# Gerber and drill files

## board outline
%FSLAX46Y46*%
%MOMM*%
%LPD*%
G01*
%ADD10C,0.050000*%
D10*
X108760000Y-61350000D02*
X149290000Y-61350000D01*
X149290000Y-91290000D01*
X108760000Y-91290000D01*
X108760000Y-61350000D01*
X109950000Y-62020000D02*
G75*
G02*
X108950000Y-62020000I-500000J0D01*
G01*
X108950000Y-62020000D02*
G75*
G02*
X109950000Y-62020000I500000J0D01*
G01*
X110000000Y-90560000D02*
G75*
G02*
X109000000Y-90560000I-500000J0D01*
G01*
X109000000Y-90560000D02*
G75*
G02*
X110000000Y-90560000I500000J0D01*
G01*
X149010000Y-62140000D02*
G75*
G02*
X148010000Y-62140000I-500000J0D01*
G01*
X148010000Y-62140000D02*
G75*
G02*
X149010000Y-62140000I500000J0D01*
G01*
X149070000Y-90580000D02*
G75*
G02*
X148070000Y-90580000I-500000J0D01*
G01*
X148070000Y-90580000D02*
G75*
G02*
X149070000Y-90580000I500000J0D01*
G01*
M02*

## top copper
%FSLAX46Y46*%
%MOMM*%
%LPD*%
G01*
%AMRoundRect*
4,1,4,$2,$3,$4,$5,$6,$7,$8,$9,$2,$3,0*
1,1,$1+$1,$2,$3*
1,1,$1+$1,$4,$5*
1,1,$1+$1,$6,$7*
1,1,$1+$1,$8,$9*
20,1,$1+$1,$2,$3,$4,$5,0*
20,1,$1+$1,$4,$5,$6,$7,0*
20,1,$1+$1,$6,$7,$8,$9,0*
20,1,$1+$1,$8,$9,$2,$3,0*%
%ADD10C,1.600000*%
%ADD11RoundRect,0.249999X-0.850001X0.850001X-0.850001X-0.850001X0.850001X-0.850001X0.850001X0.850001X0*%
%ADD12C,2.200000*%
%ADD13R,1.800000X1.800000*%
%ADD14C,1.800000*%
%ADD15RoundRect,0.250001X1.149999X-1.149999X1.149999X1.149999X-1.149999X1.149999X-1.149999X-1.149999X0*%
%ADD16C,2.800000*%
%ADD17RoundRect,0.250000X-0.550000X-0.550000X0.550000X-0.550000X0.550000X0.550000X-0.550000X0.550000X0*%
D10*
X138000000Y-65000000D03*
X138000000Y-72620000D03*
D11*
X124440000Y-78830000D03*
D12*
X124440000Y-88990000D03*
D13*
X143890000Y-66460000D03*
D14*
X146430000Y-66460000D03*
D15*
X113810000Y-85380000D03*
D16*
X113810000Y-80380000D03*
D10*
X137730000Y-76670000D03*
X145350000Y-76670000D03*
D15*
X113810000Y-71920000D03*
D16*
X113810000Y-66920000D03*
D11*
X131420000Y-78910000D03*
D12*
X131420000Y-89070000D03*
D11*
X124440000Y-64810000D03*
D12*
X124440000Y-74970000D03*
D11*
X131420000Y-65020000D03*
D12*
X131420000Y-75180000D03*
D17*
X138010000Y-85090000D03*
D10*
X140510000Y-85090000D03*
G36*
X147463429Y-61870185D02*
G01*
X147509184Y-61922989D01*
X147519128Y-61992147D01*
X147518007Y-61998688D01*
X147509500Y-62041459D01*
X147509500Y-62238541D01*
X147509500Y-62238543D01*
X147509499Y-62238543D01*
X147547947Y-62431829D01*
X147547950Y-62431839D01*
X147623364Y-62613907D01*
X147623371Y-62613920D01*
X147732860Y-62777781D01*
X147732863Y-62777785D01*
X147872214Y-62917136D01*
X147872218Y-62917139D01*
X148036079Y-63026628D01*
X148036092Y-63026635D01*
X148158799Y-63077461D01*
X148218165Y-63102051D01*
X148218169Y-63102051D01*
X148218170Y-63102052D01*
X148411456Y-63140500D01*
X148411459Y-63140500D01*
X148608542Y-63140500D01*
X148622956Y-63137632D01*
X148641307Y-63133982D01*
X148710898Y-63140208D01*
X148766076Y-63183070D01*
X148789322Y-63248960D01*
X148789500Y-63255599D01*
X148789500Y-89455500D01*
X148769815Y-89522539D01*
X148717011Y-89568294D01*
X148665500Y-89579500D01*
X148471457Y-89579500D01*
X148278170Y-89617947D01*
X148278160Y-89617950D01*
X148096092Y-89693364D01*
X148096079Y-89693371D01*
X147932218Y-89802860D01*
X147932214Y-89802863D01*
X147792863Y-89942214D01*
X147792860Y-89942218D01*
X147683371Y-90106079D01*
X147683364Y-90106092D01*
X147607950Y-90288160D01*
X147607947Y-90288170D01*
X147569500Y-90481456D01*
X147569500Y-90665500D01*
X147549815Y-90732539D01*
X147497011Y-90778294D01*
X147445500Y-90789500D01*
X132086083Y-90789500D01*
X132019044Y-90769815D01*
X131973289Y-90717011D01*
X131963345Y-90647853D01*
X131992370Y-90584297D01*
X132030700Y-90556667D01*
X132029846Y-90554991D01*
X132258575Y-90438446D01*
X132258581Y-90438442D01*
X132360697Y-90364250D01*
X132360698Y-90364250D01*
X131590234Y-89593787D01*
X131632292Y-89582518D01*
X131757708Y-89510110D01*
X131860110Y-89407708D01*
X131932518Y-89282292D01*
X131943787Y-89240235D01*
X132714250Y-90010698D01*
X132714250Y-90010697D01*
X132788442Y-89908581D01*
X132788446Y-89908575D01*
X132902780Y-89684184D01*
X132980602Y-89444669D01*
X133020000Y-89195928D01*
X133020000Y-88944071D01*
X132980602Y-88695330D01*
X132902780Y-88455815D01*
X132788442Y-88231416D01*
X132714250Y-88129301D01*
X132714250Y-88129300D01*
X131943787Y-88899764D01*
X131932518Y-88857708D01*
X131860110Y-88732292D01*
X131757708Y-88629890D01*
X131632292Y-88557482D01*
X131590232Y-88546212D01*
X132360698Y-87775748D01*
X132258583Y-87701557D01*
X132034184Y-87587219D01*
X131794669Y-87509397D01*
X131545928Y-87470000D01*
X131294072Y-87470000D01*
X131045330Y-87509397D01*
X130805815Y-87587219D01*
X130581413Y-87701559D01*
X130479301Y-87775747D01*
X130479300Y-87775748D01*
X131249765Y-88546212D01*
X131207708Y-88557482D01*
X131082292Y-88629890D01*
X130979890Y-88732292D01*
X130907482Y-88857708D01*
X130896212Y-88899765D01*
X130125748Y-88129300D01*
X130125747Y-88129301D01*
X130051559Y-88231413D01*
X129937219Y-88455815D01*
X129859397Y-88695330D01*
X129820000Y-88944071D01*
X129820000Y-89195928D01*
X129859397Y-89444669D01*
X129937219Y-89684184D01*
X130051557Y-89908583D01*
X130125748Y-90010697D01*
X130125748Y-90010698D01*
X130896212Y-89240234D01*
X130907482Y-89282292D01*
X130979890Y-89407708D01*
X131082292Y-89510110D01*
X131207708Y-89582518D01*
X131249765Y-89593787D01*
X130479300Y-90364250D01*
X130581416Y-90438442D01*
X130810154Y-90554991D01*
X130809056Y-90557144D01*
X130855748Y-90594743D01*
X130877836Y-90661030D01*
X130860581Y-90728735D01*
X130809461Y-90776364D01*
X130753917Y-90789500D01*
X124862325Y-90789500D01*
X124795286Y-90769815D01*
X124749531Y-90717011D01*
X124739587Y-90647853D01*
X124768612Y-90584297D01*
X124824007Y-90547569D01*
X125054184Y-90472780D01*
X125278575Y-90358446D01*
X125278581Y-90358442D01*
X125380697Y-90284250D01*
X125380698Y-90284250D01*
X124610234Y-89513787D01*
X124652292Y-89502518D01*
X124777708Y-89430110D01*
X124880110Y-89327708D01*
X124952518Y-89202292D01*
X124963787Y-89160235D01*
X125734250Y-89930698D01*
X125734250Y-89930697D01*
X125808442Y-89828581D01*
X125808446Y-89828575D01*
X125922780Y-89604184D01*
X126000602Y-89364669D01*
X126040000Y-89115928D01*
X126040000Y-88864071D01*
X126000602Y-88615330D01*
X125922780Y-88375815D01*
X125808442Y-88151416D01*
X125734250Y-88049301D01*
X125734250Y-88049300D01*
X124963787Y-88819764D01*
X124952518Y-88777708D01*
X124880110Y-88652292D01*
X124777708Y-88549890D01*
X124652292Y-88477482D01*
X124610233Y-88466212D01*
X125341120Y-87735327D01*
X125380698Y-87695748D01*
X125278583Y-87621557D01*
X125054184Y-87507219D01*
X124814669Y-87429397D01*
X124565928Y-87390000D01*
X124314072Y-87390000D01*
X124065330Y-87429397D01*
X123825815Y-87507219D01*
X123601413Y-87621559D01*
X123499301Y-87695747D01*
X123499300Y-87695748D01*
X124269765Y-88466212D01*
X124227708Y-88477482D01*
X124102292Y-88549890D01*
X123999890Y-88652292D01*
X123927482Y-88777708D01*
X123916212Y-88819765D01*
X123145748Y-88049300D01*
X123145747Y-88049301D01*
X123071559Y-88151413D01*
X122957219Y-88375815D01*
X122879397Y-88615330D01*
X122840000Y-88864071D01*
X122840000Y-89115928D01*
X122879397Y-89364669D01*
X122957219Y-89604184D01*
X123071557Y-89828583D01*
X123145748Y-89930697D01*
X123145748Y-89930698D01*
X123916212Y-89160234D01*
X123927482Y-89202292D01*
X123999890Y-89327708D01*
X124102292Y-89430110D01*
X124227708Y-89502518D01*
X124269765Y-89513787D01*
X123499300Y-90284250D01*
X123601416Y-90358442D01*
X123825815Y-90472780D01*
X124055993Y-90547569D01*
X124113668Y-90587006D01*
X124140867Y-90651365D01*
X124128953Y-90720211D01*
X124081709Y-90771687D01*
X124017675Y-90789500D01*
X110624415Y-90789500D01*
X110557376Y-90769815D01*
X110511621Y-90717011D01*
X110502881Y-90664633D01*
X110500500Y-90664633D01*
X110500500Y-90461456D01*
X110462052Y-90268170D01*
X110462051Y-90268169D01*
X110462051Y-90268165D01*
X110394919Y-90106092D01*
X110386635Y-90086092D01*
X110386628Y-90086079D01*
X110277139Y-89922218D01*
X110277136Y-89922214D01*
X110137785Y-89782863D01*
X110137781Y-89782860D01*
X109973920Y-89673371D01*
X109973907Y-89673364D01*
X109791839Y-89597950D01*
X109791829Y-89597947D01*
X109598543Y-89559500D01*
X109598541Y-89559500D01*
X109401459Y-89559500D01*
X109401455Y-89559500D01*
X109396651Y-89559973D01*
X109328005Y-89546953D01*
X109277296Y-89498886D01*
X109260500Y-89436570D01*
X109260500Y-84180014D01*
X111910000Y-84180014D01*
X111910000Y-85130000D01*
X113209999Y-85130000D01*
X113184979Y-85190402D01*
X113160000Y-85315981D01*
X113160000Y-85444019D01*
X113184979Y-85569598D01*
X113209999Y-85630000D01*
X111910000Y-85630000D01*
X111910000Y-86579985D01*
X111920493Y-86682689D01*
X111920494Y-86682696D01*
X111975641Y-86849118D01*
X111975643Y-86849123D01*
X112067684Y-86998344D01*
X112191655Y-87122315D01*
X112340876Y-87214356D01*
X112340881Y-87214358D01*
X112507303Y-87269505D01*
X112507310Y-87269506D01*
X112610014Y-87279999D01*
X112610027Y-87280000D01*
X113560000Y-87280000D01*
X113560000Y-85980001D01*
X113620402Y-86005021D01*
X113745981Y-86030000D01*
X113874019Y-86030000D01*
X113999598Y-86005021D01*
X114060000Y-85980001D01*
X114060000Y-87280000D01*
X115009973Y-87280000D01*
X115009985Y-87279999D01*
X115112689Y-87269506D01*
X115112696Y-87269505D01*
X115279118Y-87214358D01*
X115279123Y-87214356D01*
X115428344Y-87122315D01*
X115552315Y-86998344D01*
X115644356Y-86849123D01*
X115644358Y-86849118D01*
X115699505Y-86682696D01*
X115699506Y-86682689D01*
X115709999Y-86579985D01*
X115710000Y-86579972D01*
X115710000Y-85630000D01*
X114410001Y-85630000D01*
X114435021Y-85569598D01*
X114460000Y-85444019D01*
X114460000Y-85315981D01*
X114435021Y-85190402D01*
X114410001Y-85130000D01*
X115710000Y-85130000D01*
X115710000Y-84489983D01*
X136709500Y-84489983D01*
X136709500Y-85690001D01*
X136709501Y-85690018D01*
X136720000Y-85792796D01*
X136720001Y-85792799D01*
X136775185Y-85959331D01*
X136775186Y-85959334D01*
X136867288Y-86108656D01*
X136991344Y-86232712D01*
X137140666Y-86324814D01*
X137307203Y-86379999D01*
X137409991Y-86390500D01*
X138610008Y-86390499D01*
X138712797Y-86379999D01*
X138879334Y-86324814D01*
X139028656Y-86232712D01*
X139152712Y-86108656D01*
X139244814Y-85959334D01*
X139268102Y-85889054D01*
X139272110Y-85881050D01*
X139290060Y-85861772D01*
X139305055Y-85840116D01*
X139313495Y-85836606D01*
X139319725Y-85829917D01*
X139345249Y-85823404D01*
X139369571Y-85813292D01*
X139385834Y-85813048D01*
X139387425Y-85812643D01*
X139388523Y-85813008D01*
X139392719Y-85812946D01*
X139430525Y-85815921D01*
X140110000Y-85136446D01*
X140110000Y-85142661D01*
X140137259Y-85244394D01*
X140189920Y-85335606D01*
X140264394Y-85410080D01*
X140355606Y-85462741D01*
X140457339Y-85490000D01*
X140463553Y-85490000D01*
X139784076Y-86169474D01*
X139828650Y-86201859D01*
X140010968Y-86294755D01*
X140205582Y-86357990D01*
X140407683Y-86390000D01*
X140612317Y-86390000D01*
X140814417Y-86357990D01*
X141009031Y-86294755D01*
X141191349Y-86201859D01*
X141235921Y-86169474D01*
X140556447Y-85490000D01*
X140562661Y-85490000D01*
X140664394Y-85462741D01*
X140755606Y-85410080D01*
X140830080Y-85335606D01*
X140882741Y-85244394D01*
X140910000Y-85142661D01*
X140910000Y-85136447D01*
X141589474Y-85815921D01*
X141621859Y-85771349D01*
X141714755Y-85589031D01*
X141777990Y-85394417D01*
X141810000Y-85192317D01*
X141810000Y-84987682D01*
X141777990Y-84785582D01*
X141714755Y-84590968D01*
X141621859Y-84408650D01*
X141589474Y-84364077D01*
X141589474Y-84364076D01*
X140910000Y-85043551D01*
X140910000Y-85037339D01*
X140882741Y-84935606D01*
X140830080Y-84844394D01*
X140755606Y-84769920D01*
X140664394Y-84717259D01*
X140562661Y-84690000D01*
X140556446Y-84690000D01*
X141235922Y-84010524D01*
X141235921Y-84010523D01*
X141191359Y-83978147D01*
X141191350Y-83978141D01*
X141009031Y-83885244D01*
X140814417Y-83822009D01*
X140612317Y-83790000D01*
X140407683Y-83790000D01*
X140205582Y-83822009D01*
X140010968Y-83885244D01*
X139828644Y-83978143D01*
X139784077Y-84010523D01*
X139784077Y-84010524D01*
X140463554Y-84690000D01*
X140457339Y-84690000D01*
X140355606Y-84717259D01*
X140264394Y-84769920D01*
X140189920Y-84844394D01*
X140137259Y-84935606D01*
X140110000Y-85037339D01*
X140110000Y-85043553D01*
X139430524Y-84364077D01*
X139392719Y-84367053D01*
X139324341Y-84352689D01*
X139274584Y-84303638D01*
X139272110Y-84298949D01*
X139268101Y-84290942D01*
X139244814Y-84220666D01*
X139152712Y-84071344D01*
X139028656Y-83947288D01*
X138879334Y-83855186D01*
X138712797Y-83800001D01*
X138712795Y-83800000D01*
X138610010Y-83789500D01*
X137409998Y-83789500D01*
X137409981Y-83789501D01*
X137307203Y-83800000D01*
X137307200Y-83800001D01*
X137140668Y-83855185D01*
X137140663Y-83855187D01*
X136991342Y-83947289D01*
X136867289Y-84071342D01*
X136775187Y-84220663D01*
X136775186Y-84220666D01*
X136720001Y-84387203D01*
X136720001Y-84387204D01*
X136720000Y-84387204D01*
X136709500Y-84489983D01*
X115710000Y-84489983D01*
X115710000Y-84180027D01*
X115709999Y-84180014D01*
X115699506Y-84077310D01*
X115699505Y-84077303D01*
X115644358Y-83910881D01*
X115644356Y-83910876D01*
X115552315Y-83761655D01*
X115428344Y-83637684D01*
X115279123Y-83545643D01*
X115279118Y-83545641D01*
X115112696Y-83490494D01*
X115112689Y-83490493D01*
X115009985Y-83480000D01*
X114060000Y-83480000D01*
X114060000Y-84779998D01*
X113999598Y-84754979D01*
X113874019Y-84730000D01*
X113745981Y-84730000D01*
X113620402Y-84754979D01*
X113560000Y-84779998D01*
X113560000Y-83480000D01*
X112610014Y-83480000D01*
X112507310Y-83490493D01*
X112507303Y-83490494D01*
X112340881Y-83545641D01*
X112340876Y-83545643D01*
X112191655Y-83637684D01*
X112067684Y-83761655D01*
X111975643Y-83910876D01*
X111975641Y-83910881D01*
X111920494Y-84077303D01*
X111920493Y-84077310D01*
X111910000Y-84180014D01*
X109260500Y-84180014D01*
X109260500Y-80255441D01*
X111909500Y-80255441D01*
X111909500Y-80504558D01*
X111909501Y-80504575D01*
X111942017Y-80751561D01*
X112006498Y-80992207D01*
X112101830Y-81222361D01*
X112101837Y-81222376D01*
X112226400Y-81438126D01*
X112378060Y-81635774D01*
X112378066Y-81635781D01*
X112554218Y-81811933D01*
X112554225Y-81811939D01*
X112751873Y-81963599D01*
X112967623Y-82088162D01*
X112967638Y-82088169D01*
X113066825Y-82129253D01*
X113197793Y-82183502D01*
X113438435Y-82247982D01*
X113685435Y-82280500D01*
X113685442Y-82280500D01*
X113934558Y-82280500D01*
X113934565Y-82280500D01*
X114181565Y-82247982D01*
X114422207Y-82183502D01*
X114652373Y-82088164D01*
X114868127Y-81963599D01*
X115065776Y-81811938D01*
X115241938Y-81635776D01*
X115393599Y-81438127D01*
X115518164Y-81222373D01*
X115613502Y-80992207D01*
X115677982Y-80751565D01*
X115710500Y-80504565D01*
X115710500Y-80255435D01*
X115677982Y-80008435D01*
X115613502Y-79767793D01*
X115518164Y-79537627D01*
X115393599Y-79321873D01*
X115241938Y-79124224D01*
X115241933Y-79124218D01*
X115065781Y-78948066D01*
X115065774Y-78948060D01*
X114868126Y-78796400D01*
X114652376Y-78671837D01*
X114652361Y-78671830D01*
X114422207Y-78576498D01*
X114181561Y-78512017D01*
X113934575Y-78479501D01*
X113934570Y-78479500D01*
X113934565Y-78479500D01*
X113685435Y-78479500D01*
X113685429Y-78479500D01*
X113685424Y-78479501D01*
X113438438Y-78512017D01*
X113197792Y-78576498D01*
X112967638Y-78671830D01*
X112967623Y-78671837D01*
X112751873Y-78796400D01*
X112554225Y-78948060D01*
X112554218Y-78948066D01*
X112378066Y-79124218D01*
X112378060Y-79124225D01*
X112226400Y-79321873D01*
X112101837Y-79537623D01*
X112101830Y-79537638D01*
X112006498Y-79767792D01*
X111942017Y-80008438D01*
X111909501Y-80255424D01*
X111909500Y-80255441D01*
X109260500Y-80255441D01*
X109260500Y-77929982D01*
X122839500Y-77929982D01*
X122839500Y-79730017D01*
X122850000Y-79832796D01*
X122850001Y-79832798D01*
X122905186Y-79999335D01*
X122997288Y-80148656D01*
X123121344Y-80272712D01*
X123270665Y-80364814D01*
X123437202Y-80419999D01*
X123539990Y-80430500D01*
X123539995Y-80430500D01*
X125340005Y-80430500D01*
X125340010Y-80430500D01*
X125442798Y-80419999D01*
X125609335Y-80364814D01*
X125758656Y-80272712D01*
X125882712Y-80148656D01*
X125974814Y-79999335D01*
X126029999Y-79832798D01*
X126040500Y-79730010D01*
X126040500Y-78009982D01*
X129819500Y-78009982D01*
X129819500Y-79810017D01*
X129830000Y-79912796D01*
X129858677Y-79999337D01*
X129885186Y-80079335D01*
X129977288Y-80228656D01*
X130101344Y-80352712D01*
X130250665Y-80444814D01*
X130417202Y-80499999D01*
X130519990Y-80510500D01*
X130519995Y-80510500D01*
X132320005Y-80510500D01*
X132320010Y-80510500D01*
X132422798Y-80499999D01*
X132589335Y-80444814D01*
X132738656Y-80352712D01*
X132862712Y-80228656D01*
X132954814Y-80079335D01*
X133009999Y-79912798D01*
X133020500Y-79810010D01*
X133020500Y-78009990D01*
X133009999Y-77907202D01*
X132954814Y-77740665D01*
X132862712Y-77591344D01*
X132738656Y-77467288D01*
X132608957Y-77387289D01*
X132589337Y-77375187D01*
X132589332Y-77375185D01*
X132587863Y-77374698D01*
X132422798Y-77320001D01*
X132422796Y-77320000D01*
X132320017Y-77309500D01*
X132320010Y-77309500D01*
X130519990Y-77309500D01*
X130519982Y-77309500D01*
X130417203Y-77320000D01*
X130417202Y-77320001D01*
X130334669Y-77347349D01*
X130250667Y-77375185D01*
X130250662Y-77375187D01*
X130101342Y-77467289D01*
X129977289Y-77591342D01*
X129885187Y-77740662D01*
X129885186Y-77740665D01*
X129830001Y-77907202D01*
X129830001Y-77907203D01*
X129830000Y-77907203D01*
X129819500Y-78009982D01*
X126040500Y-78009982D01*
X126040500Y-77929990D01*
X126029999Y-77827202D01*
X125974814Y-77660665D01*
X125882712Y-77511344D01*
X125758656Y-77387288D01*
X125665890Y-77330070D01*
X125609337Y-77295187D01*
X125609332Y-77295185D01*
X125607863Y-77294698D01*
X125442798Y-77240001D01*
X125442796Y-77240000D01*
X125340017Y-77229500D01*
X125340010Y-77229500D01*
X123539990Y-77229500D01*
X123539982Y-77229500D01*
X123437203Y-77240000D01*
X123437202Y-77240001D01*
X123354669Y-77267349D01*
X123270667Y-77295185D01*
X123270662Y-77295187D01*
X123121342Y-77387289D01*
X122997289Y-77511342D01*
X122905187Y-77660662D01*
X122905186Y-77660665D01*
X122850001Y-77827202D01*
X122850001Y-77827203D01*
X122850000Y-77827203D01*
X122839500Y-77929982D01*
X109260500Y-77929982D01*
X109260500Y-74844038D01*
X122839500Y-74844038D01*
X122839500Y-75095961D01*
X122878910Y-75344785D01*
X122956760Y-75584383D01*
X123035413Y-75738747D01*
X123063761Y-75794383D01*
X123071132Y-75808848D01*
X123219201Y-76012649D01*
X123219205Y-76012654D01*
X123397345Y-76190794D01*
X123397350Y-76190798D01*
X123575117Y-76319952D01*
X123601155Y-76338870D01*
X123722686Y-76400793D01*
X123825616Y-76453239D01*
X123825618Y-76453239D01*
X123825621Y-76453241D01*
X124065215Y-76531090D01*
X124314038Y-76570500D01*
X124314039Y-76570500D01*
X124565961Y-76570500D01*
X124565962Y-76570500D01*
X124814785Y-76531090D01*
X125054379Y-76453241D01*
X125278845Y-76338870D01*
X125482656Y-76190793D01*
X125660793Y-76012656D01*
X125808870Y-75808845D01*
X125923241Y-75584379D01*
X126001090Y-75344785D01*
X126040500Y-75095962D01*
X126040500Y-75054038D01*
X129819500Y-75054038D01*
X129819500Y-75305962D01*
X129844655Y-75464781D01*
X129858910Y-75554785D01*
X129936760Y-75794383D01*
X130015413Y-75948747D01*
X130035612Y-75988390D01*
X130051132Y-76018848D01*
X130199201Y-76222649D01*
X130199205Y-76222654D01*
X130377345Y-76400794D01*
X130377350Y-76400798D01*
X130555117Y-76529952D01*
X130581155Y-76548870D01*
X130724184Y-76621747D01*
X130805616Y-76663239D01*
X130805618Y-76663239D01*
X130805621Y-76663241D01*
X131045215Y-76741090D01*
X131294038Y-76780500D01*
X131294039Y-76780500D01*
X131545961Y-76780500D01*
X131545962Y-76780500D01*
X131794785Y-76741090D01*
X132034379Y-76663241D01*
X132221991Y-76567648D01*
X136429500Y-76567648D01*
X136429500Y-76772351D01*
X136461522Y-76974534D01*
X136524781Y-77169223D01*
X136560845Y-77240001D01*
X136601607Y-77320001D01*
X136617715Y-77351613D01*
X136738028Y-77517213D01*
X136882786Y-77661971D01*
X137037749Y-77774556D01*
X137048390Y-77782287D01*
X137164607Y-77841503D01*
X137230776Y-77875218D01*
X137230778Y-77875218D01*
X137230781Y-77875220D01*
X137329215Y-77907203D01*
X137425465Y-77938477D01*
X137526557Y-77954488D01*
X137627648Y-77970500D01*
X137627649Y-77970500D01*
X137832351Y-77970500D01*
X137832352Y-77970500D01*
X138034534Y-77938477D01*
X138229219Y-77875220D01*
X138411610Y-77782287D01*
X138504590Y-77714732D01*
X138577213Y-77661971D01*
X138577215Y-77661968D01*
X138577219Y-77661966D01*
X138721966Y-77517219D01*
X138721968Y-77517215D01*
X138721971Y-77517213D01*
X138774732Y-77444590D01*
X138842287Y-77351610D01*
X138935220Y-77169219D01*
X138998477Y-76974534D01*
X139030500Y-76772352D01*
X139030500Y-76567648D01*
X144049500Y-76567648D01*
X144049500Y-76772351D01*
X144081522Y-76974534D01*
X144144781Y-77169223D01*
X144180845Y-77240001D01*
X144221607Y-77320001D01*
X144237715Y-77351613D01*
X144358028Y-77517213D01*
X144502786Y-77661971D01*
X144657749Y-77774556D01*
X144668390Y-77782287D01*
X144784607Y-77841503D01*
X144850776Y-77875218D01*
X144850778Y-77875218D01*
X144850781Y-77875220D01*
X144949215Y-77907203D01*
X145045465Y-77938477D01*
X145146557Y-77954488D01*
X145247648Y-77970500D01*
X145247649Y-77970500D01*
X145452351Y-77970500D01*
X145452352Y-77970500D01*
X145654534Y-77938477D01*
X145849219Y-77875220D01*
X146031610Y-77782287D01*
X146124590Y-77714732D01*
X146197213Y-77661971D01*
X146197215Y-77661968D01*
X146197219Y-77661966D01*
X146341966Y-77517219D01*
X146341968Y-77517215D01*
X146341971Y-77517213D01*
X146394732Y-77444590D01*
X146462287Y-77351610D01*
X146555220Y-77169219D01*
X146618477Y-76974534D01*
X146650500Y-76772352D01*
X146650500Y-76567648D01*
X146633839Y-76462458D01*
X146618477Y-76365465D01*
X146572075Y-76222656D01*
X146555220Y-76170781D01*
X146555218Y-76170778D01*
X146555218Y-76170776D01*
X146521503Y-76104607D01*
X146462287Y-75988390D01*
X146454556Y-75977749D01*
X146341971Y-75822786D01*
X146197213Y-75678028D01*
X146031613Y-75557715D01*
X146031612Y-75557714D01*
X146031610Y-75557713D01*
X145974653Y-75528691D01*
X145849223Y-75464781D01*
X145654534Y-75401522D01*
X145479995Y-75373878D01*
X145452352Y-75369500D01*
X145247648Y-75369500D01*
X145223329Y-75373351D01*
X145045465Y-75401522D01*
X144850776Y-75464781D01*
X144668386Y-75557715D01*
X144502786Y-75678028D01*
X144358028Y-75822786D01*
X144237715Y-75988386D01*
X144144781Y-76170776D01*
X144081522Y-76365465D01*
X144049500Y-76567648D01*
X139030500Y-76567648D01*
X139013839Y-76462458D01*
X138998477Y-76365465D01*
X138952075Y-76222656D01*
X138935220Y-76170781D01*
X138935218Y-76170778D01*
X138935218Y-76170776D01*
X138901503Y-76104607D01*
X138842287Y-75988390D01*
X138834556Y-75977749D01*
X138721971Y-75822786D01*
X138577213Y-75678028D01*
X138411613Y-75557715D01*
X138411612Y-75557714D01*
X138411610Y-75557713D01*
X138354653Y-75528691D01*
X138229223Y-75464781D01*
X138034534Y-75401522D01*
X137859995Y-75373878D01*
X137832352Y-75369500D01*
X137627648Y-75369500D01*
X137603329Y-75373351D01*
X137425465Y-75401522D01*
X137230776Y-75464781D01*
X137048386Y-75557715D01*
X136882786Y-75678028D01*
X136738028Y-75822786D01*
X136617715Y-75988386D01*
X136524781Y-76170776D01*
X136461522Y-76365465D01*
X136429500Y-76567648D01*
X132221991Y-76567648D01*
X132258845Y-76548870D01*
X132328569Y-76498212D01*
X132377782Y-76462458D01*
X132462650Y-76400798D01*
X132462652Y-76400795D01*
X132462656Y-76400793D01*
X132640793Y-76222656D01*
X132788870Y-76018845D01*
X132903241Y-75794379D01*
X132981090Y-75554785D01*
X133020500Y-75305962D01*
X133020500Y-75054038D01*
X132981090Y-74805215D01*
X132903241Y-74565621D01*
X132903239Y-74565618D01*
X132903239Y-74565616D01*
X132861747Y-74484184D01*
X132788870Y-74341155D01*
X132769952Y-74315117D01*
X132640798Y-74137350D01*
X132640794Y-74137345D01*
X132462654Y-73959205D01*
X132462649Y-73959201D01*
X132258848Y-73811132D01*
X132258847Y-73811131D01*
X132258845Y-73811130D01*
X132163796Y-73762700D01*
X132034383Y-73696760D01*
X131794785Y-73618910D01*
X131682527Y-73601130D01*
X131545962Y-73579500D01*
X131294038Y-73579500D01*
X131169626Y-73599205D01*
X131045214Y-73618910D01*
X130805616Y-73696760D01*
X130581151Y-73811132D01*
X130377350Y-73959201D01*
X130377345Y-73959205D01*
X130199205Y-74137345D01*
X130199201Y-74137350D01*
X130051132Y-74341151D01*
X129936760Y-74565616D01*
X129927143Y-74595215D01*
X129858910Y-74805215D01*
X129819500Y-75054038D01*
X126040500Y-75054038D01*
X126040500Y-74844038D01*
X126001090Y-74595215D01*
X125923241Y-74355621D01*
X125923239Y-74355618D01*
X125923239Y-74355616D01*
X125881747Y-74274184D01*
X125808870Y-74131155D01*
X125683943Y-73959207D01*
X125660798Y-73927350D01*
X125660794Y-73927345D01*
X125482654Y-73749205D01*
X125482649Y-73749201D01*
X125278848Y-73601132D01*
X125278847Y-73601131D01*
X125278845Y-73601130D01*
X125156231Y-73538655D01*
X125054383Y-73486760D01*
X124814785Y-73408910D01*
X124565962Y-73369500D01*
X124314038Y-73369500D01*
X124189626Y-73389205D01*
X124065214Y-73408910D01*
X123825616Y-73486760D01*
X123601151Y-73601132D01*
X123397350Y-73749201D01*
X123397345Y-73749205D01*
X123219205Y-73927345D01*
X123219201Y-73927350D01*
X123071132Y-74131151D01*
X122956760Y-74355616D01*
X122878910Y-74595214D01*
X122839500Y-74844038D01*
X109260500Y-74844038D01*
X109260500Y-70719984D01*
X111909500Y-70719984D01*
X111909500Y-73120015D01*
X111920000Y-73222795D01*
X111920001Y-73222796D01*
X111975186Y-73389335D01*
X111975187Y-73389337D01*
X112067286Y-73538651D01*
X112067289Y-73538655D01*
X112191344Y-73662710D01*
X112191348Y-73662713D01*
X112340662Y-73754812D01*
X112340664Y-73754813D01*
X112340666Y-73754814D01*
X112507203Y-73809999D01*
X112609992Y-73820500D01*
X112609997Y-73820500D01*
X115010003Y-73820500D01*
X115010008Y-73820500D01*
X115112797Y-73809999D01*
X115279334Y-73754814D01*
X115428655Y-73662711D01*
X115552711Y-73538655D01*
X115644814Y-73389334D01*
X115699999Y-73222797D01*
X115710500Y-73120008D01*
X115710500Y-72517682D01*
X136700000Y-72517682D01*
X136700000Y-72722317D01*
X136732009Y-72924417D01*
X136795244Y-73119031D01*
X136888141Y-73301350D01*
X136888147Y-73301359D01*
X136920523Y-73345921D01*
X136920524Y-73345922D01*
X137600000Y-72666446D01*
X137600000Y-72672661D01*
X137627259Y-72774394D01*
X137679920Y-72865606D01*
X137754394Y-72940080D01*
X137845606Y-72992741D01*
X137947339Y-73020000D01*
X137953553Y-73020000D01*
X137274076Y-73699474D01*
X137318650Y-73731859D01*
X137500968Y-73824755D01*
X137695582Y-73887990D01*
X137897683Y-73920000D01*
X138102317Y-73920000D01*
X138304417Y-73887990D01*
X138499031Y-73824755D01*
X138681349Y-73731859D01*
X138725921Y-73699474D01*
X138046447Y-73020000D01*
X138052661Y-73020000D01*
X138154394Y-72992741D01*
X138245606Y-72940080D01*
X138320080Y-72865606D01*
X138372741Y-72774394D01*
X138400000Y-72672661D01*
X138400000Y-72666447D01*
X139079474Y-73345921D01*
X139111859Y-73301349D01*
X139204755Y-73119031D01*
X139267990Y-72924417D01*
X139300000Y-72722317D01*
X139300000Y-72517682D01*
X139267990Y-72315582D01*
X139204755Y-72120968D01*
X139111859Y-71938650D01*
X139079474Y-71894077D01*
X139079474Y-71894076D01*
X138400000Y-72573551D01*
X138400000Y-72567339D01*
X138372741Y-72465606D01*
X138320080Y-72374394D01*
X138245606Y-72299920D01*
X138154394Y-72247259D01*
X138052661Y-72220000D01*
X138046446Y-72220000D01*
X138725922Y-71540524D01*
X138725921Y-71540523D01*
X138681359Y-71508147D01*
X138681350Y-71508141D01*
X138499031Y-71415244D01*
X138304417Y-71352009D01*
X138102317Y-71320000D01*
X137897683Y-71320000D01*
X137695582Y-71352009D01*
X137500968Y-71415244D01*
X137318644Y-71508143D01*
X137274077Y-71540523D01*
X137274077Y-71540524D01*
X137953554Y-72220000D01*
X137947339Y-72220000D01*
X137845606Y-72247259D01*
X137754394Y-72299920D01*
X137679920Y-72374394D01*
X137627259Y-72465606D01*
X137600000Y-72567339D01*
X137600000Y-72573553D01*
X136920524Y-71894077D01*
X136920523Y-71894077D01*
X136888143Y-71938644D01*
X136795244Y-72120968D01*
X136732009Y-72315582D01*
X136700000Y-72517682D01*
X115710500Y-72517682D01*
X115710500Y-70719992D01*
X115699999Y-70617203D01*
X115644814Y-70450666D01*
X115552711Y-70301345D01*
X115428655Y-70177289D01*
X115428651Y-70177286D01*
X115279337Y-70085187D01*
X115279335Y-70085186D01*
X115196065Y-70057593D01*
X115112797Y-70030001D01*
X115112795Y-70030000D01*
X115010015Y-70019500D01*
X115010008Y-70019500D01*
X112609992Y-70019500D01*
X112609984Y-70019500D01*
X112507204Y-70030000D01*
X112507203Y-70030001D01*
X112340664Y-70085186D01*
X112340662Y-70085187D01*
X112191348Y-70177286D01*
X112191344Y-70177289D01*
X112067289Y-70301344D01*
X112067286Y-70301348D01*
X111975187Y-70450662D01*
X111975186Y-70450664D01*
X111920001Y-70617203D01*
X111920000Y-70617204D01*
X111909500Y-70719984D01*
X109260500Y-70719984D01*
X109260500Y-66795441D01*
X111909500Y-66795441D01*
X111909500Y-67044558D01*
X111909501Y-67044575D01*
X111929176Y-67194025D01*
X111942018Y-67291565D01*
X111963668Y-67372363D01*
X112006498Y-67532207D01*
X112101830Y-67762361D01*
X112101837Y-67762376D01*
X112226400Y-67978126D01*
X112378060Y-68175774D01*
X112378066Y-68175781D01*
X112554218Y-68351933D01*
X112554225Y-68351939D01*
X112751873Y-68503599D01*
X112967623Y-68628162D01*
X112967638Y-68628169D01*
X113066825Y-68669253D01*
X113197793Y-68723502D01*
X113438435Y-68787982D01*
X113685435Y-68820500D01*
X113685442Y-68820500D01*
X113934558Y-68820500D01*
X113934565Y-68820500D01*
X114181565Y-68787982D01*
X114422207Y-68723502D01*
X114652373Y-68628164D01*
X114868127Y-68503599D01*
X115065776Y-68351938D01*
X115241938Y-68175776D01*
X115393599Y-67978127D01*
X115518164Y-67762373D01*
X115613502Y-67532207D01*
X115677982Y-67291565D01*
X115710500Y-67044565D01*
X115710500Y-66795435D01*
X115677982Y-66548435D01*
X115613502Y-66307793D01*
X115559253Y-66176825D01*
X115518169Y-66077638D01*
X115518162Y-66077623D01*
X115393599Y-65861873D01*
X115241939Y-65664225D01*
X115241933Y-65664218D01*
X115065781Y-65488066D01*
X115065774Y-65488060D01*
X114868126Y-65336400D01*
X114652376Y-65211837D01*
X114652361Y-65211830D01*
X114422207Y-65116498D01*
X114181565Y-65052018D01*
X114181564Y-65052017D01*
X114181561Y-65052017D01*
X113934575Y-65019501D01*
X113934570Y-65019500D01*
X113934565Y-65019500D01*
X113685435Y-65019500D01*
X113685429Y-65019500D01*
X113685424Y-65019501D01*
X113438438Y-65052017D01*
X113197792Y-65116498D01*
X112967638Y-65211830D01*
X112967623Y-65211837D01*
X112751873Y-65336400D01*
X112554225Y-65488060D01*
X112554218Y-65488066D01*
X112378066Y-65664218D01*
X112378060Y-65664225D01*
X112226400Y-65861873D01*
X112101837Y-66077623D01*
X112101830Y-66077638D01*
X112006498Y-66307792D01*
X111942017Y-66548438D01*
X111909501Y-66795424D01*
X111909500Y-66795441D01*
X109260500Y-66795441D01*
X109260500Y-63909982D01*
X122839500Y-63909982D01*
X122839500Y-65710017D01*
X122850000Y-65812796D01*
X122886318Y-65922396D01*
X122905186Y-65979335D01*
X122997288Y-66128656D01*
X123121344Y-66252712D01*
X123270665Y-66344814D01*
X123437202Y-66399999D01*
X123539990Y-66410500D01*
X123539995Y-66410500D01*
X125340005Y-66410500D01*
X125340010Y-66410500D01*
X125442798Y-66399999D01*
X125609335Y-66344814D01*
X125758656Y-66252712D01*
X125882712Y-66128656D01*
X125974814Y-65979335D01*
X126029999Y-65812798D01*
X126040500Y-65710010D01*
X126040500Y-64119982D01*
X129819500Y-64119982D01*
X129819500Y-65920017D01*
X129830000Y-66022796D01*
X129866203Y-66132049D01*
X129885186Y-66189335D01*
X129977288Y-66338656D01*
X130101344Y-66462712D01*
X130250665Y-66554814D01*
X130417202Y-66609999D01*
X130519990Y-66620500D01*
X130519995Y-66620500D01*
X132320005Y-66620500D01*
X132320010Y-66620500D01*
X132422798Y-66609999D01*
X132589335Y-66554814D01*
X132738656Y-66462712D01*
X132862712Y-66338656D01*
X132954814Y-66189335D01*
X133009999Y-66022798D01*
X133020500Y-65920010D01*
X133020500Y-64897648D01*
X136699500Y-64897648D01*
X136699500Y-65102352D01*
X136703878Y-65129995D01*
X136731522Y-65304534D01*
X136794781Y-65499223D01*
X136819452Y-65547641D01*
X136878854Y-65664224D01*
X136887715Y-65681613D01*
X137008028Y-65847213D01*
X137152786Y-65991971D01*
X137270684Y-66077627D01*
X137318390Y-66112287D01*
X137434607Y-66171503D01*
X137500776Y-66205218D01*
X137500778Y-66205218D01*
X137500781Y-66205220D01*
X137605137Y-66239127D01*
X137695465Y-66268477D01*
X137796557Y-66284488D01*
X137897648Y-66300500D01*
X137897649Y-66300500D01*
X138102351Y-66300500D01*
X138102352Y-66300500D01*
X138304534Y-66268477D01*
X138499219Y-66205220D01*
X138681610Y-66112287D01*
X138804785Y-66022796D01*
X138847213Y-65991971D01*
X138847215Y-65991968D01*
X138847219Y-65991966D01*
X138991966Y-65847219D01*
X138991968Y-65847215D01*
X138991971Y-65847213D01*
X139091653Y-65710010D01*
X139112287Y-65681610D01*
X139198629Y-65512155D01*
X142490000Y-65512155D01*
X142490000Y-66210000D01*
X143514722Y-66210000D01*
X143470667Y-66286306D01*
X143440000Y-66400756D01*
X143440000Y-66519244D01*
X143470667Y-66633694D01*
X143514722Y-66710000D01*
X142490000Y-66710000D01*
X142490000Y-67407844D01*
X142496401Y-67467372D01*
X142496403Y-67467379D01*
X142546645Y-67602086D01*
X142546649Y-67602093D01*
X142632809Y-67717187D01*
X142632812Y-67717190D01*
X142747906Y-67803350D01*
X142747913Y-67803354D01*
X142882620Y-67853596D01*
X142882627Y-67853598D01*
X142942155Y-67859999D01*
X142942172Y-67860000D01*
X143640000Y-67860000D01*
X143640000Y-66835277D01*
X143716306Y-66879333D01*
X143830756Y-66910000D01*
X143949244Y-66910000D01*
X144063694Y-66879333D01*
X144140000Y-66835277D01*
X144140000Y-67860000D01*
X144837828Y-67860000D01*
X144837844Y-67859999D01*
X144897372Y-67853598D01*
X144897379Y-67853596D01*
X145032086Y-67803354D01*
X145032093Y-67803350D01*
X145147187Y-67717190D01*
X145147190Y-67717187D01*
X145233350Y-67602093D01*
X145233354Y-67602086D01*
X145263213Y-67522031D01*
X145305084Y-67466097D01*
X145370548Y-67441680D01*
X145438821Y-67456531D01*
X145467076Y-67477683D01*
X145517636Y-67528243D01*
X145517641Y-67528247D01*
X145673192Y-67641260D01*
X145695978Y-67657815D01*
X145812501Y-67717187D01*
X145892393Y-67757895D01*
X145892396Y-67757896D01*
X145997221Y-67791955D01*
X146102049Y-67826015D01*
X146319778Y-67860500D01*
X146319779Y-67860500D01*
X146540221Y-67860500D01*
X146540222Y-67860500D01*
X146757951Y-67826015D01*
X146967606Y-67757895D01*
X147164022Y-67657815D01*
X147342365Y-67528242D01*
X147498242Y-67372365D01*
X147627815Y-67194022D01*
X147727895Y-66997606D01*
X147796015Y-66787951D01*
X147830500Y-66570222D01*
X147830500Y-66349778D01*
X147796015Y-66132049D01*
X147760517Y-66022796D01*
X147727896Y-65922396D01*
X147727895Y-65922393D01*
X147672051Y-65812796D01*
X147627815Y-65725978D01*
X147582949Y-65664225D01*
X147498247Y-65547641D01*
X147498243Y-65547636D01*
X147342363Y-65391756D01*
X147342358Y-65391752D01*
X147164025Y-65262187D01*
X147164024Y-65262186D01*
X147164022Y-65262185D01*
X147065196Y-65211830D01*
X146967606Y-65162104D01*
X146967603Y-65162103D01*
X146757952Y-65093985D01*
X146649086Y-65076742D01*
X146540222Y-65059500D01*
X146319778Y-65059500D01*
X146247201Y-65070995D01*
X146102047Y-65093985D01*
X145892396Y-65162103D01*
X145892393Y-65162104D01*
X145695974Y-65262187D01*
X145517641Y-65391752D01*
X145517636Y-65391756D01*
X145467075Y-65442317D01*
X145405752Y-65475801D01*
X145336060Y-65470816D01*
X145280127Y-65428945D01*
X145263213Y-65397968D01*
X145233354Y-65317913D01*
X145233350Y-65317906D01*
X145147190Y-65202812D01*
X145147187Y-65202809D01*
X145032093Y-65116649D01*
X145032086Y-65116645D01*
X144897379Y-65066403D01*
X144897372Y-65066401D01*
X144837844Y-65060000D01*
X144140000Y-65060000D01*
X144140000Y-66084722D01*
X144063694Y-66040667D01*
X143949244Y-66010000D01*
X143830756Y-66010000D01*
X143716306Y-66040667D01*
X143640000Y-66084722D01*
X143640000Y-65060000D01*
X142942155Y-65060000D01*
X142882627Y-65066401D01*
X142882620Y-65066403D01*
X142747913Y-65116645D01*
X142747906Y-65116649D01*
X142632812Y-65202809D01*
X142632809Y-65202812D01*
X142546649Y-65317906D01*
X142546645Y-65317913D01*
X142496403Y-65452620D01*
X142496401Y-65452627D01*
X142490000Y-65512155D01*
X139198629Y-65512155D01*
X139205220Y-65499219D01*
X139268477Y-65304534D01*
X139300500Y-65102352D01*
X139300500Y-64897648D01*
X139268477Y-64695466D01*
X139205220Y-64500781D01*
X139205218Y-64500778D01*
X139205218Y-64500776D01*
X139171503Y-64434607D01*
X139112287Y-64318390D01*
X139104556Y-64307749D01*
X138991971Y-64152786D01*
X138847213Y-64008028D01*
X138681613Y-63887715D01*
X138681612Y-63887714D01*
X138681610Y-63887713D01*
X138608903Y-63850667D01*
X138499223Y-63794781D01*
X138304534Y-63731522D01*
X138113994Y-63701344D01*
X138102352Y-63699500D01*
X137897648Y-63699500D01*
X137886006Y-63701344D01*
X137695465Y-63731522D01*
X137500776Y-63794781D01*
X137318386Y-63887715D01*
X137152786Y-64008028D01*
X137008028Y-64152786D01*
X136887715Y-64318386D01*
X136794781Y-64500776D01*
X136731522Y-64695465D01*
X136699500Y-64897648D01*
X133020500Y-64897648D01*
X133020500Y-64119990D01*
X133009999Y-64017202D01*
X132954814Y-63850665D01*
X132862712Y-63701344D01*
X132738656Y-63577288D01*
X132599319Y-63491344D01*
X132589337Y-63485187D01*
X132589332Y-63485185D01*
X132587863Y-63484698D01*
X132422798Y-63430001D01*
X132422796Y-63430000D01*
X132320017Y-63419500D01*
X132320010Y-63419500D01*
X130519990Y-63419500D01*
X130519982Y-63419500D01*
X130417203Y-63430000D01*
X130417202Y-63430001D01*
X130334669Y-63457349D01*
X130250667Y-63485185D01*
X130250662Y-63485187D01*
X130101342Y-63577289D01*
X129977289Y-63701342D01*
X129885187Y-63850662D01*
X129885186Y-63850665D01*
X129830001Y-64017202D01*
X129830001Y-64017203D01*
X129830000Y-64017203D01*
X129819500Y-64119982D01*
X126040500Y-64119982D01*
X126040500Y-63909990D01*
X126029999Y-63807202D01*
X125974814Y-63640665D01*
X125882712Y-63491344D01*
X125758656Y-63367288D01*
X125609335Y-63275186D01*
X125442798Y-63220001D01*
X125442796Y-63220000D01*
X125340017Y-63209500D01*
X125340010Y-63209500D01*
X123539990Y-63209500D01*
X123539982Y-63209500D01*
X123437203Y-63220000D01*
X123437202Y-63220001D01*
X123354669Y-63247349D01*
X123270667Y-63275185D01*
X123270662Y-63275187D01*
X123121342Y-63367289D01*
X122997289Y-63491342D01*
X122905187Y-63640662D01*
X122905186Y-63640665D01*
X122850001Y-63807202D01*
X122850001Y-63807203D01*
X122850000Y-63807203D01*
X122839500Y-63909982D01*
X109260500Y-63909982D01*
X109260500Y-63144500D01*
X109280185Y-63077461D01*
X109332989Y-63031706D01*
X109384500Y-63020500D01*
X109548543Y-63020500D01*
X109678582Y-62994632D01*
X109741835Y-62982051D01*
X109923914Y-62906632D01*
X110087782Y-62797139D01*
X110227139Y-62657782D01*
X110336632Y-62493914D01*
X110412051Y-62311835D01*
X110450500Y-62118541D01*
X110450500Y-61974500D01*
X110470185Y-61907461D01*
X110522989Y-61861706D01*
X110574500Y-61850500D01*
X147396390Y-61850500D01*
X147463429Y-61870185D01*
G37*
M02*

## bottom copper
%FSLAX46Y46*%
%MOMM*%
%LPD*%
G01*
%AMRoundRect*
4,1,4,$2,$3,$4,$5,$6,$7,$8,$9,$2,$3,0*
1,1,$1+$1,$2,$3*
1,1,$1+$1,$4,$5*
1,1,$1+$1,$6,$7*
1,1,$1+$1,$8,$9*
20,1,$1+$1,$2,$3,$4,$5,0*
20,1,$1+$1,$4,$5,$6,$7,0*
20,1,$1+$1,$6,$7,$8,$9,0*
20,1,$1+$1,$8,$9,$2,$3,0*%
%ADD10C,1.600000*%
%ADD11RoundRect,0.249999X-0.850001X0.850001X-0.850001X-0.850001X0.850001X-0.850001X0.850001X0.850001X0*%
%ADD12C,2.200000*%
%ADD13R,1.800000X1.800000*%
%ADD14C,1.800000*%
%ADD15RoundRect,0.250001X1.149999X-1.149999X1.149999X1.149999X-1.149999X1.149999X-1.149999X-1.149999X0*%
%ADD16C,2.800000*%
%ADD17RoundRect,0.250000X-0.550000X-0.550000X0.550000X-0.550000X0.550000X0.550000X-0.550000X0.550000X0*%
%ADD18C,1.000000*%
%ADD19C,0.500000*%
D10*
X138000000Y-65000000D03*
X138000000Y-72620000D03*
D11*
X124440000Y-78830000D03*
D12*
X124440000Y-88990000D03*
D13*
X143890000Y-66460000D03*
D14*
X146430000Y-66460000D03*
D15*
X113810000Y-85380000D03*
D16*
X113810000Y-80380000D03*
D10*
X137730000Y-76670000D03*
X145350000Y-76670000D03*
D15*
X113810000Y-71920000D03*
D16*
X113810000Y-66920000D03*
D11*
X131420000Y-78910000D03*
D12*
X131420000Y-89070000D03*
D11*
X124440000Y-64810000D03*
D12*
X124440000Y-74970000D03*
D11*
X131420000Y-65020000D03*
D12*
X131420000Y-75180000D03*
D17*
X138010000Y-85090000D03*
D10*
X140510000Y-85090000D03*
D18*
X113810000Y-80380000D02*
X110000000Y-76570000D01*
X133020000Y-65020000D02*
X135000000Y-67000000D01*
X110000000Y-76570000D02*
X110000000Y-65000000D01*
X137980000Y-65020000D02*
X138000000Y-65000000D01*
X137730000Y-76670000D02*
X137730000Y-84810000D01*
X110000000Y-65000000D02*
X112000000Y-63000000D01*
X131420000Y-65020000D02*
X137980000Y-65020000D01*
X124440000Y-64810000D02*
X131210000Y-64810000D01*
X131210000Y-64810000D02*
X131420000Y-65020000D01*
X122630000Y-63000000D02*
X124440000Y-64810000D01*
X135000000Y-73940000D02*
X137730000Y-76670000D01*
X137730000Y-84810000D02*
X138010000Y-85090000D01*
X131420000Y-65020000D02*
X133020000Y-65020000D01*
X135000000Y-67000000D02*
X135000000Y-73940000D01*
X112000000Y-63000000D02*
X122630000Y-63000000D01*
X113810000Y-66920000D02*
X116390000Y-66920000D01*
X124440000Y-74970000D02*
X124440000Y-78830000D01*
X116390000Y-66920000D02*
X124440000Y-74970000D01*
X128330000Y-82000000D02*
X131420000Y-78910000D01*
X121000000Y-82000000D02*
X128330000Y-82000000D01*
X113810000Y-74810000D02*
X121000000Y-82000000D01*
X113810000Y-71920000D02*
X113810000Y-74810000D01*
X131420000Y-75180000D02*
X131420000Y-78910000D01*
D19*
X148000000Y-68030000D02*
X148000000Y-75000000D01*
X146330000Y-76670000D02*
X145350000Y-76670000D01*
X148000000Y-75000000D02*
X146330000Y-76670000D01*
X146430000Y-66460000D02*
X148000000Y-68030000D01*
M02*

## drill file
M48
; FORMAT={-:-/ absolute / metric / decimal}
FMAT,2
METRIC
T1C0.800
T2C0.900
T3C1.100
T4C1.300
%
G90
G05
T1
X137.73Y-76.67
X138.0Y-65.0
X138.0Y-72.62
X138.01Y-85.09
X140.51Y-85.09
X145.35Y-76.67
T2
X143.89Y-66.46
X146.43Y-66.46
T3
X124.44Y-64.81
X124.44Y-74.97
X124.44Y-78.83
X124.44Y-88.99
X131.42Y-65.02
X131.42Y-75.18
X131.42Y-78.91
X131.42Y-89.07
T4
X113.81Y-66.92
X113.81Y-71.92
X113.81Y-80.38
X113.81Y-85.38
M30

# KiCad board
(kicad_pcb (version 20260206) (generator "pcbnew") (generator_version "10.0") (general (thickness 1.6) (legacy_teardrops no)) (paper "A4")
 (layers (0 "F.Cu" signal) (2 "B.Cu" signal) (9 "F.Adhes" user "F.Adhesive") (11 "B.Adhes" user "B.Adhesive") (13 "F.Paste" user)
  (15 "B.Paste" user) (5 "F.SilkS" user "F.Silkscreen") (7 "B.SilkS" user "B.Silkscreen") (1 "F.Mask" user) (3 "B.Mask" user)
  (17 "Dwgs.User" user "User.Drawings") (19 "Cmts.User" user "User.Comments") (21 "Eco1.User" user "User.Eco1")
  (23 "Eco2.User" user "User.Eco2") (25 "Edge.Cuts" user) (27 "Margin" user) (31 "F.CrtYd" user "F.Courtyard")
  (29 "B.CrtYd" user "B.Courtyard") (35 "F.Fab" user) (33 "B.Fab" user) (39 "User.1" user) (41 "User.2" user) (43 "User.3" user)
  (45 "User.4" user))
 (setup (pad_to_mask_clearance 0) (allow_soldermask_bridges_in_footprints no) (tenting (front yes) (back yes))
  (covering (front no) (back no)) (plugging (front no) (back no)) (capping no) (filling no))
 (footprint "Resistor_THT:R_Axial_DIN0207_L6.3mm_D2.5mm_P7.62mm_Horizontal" (layer "F.Cu") (at 138 65 -90)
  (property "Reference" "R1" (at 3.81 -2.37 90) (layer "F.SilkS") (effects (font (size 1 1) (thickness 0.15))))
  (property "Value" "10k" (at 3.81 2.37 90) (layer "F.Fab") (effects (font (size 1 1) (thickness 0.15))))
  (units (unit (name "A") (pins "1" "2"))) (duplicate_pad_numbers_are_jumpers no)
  (pad "1" thru_hole circle (at 0 0 270) (size 1.6 1.6) (drill 0.8) (layers "*.Cu" "*.Mask") (remove_unused_layers no) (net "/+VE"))
  (pad "2" thru_hole circle (at 7.62 0 270) (size 1.6 1.6) (drill 0.8) (layers "*.Cu" "*.Mask") (remove_unused_layers no) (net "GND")))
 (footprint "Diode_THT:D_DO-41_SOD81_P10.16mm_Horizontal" (layer "F.Cu") (at 124.44 78.83 -90)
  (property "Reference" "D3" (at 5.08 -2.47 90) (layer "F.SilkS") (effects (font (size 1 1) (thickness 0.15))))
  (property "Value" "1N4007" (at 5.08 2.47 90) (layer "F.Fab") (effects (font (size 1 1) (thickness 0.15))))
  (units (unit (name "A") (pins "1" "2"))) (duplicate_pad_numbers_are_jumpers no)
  (pad "1" thru_hole roundrect (at 0 0 270) (size 2.2 2.2) (drill 1.1) (layers "*.Cu" "*.Mask") (remove_unused_layers no)
   (roundrect_rratio 0.113636) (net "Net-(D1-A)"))
  (pad "2" thru_hole circle (at 10.16 0 270) (size 2.2 2.2) (drill 1.1) (layers "*.Cu" "*.Mask") (remove_unused_layers no) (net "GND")))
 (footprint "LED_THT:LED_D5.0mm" (layer "F.Cu") (at 143.89 66.46)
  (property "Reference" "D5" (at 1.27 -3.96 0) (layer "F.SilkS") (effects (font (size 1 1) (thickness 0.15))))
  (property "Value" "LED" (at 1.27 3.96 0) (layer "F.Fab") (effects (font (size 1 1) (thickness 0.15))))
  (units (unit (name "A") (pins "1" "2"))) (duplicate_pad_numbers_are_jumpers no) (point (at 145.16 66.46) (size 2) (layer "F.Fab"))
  (pad "1" thru_hole rect (at 0 0) (size 1.8 1.8) (drill 0.9) (layers "*.Cu" "*.Mask") (remove_unused_layers no) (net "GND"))
  (pad "2" thru_hole circle (at 2.54 0) (size 1.8 1.8) (drill 0.9) (layers "*.Cu" "*.Mask") (remove_unused_layers no) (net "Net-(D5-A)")))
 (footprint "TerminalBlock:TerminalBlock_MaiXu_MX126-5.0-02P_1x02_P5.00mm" (layer "F.Cu") (at 113.81 85.38 90)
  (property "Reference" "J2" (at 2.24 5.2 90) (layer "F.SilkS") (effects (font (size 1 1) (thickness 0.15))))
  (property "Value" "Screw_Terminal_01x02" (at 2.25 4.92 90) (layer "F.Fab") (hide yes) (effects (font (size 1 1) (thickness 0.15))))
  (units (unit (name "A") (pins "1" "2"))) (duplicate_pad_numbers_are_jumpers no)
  (pad "1" thru_hole roundrect (at 0 0 90) (size 2.8 2.8) (drill 1.3) (layers "*.Cu" "*.Mask") (remove_unused_layers no)
   (roundrect_rratio 0.089286) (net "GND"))
  (pad "2" thru_hole circle (at 5 0 90) (size 2.8 2.8) (drill 1.3) (layers "*.Cu" "*.Mask") (remove_unused_layers no) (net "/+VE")))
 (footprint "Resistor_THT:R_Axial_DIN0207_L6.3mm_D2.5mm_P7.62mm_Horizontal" (layer "F.Cu") (at 137.73 76.67)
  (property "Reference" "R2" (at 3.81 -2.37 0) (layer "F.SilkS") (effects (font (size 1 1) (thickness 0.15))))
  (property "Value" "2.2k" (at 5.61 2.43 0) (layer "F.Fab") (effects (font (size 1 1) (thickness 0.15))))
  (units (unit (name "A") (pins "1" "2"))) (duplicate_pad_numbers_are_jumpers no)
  (pad "1" thru_hole circle (at 0 0) (size 1.6 1.6) (drill 0.8) (layers "*.Cu" "*.Mask") (remove_unused_layers no) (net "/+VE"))
  (pad "2" thru_hole circle (at 7.62 0) (size 1.6 1.6) (drill 0.8) (layers "*.Cu" "*.Mask") (remove_unused_layers no) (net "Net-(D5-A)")))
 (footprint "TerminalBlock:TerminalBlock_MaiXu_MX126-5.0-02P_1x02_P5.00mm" (layer "F.Cu") (at 113.81 71.92 90)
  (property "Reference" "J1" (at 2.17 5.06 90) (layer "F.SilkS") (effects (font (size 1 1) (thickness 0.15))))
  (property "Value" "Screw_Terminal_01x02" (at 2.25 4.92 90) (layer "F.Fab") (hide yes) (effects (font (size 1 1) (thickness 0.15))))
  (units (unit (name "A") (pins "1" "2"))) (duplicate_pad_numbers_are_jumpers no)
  (pad "1" thru_hole roundrect (at 0 0 90) (size 2.8 2.8) (drill 1.3) (layers "*.Cu" "*.Mask") (remove_unused_layers no)
   (roundrect_rratio 0.089286) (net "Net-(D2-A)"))
  (pad "2" thru_hole circle (at 5 0 90) (size 2.8 2.8) (drill 1.3) (layers "*.Cu" "*.Mask") (remove_unused_layers no) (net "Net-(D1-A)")))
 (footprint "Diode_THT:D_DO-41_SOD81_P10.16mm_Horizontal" (layer "F.Cu") (at 131.42 78.91 -90)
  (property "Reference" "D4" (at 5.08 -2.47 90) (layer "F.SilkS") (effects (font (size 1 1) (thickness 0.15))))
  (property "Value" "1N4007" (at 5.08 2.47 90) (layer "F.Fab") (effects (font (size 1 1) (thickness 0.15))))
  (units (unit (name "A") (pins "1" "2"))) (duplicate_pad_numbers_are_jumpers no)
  (pad "1" thru_hole roundrect (at 0 0 270) (size 2.2 2.2) (drill 1.1) (layers "*.Cu" "*.Mask") (remove_unused_layers no)
   (roundrect_rratio 0.113636) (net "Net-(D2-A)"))
  (pad "2" thru_hole circle (at 10.16 0 270) (size 2.2 2.2) (drill 1.1) (layers "*.Cu" "*.Mask") (remove_unused_layers no) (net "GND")))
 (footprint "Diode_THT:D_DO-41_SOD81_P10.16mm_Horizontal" (layer "F.Cu") (at 124.44 64.81 -90)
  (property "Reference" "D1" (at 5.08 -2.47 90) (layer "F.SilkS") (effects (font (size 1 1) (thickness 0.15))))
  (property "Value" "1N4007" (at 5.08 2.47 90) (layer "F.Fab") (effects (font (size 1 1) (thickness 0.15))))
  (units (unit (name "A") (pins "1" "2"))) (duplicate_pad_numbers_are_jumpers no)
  (pad "1" thru_hole roundrect (at 0 0 270) (size 2.2 2.2) (drill 1.1) (layers "*.Cu" "*.Mask") (remove_unused_layers no)
   (roundrect_rratio 0.113636) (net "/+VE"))
  (pad "2" thru_hole circle (at 10.16 0 270) (size 2.2 2.2) (drill 1.1) (layers "*.Cu" "*.Mask") (remove_unused_layers no)
   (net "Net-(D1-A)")))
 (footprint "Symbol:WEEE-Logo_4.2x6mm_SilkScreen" (layer "F.Cu") (at 145.91 85.12)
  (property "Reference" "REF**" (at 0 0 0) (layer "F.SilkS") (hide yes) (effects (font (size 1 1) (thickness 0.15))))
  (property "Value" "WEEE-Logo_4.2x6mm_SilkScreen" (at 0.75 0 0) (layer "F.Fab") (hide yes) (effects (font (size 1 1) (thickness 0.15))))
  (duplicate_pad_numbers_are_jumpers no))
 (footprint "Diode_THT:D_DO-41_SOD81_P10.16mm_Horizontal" (layer "F.Cu") (at 131.42 65.02 -90)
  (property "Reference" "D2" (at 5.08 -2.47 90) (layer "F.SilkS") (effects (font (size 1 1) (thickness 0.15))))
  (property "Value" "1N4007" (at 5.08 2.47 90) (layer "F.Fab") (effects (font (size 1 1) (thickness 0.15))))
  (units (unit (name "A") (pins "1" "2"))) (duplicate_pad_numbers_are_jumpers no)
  (pad "1" thru_hole roundrect (at 0 0 270) (size 2.2 2.2) (drill 1.1) (layers "*.Cu" "*.Mask") (remove_unused_layers no)
   (roundrect_rratio 0.113636) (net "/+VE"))
  (pad "2" thru_hole circle (at 10.16 0 270) (size 2.2 2.2) (drill 1.1) (layers "*.Cu" "*.Mask") (remove_unused_layers no)
   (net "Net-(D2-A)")))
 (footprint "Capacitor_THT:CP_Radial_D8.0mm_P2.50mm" (layer "F.Cu") (at 138.01 85.09)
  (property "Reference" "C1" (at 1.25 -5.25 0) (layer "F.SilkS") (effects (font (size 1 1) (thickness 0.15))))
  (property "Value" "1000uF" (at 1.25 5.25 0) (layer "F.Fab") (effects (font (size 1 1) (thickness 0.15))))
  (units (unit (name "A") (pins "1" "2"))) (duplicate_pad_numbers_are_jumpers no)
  (pad "1" thru_hole roundrect (at 0 0) (size 1.6 1.6) (drill 0.8) (layers "*.Cu" "*.Mask") (remove_unused_layers no)
   (roundrect_rratio 0.15625) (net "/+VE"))
  (pad "2" thru_hole circle (at 2.5 0) (size 1.6 1.6) (drill 0.8) (layers "*.Cu" "*.Mask") (remove_unused_layers no) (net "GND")))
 (gr_rect (start 108.76 61.35) (end 149.29 91.29) (stroke (width 0.05) (type default)) (fill no) (layer "Edge.Cuts"))
 (gr_circle (center 109.45 62.02) (end 109.95 62.02) (stroke (width 0.05) (type solid)) (fill no) (layer "Edge.Cuts"))
 (gr_circle (center 109.5 90.56) (end 110 90.56) (stroke (width 0.05) (type solid)) (fill no) (layer "Edge.Cuts"))
 (gr_circle (center 148.51 62.14) (end 149.01 62.14) (stroke (width 0.05) (type solid)) (fill no) (layer "Edge.Cuts"))
 (gr_circle (center 148.57 90.58) (end 149.07 90.58) (stroke (width 0.05) (type solid)) (fill no) (layer "Edge.Cuts"))
 (segment (start 113.81 80.38) (end 110 76.57) (width 1) (layer "B.Cu") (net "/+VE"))
 (segment (start 133.02 65.02) (end 135 67) (width 1) (layer "B.Cu") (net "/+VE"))
 (segment (start 110 76.57) (end 110 65) (width 1) (layer "B.Cu") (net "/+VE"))
 (segment (start 137.98 65.02) (end 138 65) (width 1) (layer "B.Cu") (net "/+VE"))
 (segment (start 137.73 76.67) (end 137.73 84.81) (width 1) (layer "B.Cu") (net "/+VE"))
 (segment (start 110 65) (end 112 63) (width 1) (layer "B.Cu") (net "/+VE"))
 (segment (start 131.42 65.02) (end 137.98 65.02) (width 1) (layer "B.Cu") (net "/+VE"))
 (segment (start 124.44 64.81) (end 131.21 64.81) (width 1) (layer "B.Cu") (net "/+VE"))
 (segment (start 131.21 64.81) (end 131.42 65.02) (width 1) (layer "B.Cu") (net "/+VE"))
 (segment (start 122.63 63) (end 124.44 64.81) (width 1) (layer "B.Cu") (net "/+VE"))
 (segment (start 135 73.94) (end 137.73 76.67) (width 1) (layer "B.Cu") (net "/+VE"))
 (segment (start 137.73 84.81) (end 138.01 85.09) (width 1) (layer "B.Cu") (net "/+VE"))
 (segment (start 131.42 65.02) (end 133.02 65.02) (width 1) (layer "B.Cu") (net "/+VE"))
 (segment (start 135 67) (end 135 73.94) (width 1) (layer "B.Cu") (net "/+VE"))
 (segment (start 112 63) (end 122.63 63) (width 1) (layer "B.Cu") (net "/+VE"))
 (segment (start 113.81 66.92) (end 116.39 66.92) (width 1) (layer "B.Cu") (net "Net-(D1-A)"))
 (segment (start 124.44 74.97) (end 124.44 78.83) (width 1) (layer "B.Cu") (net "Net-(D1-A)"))
 (segment (start 116.39 66.92) (end 124.44 74.97) (width 1) (layer "B.Cu") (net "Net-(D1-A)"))
 (segment (start 128.33 82) (end 131.42 78.91) (width 1) (layer "B.Cu") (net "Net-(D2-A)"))
 (segment (start 121 82) (end 128.33 82) (width 1) (layer "B.Cu") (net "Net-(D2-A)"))
 (segment (start 113.81 74.81) (end 121 82) (width 1) (layer "B.Cu") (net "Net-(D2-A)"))
 (segment (start 113.81 71.92) (end 113.81 74.81) (width 1) (layer "B.Cu") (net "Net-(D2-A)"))
 (segment (start 131.42 75.18) (end 131.42 78.91) (width 1) (layer "B.Cu") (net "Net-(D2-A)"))
 (segment (start 148 68.03) (end 148 75) (width 0.5) (layer "B.Cu") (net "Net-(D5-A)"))
 (segment (start 146.33 76.67) (end 145.35 76.67) (width 0.5) (layer "B.Cu") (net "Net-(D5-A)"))
 (segment (start 148 75) (end 146.33 76.67) (width 0.5) (layer "B.Cu") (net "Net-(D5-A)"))
 (segment (start 146.43 66.46) (end 148 68.03) (width 0.5) (layer "B.Cu") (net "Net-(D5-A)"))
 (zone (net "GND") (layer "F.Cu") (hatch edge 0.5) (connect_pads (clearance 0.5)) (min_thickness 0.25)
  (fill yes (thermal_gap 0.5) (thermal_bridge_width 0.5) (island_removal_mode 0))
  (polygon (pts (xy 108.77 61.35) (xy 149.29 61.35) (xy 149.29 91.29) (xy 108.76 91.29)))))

